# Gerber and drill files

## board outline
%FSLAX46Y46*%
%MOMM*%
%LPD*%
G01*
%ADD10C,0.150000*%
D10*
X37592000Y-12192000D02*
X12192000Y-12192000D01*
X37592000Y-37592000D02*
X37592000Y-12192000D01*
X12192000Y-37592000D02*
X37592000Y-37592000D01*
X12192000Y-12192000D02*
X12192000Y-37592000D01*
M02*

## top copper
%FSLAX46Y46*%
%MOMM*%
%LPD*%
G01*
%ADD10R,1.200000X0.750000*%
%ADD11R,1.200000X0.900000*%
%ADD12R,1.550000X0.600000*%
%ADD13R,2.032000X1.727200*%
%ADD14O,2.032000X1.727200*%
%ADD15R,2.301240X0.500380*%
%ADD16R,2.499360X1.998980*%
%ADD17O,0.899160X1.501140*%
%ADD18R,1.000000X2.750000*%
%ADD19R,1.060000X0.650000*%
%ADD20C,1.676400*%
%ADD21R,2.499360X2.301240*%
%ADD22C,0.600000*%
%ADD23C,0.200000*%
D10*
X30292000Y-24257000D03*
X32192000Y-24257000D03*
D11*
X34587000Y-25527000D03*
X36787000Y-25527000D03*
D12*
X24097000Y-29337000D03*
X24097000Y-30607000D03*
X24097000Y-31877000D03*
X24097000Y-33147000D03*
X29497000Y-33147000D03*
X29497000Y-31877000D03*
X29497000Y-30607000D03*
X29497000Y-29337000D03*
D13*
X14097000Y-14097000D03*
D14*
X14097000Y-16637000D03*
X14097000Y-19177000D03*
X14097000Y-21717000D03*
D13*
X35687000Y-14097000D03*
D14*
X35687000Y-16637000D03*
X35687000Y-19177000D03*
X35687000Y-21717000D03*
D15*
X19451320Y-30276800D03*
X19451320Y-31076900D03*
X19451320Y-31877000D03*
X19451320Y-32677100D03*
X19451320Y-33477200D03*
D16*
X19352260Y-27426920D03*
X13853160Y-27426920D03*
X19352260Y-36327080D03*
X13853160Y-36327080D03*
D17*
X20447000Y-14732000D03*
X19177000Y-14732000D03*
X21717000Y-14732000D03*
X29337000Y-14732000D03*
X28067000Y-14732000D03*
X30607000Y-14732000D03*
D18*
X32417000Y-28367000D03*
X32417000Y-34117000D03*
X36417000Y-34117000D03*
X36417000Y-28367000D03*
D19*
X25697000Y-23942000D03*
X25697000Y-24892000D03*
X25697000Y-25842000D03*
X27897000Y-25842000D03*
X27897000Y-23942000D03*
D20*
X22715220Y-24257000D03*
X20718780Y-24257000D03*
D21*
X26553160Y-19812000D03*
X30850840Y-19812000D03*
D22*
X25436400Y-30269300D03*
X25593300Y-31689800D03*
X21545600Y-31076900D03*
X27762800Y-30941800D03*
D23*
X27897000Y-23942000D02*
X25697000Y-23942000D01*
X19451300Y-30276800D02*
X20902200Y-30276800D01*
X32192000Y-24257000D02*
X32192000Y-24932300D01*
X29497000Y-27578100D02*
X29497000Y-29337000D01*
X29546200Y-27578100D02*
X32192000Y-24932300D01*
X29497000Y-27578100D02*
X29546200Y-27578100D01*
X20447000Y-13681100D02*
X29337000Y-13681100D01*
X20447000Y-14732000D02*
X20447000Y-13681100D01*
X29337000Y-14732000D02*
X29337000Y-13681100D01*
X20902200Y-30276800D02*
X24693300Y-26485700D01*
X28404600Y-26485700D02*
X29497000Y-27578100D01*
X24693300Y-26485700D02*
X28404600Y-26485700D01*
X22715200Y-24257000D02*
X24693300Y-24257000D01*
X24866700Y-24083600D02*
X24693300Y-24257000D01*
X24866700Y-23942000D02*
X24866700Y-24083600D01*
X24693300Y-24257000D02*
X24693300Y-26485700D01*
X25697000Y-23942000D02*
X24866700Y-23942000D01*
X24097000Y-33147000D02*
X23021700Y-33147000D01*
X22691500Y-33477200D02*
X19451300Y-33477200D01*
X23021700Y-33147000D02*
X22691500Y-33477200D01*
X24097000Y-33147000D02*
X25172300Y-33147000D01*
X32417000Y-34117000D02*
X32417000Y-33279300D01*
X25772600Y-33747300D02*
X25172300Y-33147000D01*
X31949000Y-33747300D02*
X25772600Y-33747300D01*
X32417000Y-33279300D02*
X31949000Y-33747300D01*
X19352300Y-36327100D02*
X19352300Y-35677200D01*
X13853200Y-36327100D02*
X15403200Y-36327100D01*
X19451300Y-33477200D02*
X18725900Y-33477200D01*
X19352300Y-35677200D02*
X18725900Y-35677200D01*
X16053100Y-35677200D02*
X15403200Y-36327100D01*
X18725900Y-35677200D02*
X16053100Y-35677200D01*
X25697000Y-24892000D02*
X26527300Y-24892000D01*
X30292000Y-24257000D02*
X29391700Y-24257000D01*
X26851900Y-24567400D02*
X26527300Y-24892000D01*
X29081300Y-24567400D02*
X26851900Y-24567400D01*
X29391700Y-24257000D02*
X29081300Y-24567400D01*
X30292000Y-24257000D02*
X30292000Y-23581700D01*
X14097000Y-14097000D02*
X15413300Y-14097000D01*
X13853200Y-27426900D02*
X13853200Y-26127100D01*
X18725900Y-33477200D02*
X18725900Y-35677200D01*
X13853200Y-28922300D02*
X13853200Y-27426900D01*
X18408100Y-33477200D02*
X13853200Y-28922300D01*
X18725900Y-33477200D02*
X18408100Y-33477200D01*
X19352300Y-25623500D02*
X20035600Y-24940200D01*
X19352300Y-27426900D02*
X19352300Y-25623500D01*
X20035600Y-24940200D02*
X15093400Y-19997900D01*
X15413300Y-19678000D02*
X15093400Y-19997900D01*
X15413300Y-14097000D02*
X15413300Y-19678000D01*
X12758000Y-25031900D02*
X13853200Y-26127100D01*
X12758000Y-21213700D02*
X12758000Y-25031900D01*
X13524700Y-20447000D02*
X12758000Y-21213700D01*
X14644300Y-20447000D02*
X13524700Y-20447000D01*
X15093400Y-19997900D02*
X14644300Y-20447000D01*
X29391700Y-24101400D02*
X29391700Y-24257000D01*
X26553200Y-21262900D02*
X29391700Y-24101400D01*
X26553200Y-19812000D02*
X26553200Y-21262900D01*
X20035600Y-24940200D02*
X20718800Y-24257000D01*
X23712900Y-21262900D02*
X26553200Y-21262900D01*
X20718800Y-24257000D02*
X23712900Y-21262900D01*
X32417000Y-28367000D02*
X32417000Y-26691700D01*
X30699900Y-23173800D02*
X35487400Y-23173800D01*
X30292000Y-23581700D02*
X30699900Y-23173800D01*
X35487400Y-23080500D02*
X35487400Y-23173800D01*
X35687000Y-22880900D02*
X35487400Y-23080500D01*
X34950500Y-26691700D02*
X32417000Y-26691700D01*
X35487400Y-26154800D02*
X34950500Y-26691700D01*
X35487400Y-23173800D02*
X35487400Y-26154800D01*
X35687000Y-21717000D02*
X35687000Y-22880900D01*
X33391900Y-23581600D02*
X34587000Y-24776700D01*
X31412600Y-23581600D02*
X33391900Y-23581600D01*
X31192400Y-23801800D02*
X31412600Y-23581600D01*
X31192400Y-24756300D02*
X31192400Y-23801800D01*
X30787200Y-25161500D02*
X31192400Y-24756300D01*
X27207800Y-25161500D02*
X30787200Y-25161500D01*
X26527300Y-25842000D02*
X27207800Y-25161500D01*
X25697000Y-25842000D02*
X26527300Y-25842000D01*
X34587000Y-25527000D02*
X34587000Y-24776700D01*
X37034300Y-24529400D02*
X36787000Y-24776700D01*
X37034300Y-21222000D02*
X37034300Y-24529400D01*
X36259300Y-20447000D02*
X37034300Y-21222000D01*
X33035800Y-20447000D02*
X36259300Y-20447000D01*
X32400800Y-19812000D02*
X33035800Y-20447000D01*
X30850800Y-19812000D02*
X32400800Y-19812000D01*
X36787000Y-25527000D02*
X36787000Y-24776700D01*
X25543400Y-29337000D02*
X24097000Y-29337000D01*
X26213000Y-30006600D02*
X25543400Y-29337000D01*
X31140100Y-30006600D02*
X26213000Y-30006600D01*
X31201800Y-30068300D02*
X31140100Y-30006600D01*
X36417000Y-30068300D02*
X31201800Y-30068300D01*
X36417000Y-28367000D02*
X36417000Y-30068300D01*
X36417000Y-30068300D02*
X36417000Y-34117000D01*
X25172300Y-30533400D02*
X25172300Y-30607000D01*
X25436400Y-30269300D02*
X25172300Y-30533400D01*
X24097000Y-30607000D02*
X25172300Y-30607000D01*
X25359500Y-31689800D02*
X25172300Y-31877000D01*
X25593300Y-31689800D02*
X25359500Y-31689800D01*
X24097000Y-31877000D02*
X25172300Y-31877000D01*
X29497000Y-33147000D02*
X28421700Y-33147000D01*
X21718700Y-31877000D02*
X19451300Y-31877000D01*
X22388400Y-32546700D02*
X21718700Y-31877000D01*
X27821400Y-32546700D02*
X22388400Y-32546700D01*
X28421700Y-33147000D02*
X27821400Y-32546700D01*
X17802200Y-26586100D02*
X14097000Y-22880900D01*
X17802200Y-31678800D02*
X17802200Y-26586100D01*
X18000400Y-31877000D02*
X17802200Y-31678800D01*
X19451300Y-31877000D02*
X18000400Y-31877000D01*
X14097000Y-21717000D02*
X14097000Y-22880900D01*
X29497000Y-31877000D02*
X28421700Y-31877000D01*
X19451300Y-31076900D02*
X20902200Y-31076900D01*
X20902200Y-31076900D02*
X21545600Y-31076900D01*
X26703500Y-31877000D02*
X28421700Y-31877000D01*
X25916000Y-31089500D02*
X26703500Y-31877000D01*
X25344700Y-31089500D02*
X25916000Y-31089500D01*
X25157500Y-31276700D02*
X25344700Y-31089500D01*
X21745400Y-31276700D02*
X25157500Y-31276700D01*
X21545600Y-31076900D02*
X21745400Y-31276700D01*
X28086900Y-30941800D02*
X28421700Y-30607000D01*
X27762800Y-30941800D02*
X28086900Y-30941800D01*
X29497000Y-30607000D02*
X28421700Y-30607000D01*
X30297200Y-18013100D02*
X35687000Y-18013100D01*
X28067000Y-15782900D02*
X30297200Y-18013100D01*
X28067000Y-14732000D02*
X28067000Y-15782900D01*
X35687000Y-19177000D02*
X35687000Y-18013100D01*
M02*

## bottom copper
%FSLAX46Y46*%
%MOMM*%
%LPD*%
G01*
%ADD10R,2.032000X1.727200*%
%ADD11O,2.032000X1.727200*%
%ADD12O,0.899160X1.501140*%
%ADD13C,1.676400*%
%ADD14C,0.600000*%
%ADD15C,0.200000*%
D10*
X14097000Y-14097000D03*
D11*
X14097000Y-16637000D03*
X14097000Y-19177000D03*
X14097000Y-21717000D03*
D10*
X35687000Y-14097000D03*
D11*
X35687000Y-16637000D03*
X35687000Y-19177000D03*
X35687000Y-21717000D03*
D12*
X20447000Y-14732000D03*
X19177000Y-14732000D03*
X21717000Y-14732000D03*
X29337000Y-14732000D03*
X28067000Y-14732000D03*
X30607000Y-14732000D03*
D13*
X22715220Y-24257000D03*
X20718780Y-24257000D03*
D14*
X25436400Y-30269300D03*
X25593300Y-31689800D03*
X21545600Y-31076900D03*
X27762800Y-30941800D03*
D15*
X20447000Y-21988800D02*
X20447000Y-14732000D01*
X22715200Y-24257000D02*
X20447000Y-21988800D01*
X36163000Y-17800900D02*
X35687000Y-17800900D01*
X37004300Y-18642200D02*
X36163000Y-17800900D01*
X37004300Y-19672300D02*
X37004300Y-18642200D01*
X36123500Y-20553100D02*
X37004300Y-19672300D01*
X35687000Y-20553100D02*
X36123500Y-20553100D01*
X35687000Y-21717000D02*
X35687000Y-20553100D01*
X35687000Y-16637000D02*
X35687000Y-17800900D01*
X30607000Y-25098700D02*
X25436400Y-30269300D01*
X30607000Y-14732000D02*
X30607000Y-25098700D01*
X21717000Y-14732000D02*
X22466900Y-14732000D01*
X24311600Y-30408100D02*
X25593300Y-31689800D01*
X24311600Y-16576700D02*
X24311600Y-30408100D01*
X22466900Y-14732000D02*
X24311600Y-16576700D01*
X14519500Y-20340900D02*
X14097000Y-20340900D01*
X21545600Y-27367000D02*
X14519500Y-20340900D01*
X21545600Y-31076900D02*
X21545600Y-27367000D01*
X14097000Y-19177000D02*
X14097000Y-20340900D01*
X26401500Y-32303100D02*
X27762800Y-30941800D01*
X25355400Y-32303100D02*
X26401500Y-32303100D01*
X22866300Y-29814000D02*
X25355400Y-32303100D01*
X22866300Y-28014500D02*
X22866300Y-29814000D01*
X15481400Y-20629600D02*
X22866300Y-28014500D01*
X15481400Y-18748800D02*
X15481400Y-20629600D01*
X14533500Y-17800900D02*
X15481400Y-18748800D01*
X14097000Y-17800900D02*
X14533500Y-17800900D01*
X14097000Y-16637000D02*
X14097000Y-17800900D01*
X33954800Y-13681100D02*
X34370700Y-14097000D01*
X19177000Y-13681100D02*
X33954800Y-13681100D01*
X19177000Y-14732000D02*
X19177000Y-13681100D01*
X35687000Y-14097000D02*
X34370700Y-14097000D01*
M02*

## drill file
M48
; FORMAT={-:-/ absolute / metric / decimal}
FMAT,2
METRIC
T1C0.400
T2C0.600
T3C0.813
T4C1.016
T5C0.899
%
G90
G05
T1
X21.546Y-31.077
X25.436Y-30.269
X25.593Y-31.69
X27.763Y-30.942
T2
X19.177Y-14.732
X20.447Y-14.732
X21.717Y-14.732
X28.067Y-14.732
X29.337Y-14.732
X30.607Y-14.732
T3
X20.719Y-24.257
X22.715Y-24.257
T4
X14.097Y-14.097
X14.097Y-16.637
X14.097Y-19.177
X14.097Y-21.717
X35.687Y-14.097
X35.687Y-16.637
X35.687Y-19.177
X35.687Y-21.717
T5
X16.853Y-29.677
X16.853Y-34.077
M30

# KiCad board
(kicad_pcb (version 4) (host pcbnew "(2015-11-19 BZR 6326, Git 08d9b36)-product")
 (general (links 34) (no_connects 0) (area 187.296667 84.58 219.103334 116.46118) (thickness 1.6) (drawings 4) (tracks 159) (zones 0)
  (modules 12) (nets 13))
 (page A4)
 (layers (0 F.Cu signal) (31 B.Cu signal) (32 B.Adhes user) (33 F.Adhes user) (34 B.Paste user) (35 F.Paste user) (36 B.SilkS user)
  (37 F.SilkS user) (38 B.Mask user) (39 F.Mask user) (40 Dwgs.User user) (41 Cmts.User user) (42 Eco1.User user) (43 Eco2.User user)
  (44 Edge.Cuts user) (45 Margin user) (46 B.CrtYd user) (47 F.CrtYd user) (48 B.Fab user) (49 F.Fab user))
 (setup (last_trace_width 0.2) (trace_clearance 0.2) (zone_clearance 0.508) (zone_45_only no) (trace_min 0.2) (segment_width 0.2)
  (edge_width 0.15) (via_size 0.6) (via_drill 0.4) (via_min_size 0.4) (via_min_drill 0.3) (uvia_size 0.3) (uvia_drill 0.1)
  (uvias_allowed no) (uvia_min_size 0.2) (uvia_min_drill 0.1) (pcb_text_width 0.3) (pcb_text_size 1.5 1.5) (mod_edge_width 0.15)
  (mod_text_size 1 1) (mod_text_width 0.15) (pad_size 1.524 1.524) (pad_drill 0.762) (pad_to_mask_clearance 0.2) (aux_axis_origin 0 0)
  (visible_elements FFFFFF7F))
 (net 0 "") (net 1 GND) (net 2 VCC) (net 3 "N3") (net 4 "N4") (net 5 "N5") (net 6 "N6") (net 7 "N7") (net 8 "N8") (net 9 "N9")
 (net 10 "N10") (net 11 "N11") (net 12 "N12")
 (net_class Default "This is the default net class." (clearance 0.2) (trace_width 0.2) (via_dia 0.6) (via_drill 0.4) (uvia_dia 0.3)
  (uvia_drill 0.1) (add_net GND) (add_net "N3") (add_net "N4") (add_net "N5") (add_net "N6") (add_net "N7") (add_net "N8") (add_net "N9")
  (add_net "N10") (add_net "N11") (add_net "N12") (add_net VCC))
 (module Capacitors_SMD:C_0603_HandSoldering (layer F.Cu) (at 31.242 24.257)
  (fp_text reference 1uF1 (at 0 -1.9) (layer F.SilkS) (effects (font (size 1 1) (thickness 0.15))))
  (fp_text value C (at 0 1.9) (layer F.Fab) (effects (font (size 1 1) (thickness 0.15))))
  (pad 1 smd rect (at -0.95 0) (size 1.2 0.75) (layers F.Cu F.Paste F.Mask) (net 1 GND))
  (pad 2 smd rect (at 0.95 0) (size 1.2 0.75) (layers F.Cu F.Paste F.Mask) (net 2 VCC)))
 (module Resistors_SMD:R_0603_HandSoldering (layer F.Cu) (at 35.687 25.527)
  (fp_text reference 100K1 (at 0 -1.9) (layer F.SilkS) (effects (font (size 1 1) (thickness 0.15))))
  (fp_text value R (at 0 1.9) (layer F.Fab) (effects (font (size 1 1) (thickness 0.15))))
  (pad 1 smd rect (at -1.1 0) (size 1.2 0.9) (layers F.Cu F.Paste F.Mask) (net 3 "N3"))
  (pad 2 smd rect (at 1.1 0) (size 1.2 0.9) (layers F.Cu F.Paste F.Mask) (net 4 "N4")))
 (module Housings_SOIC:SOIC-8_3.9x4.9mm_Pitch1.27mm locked (layer F.Cu) (at 26.797 31.242)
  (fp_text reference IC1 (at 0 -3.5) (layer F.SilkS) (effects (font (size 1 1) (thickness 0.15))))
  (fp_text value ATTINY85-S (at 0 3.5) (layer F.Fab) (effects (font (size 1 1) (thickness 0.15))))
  (pad 1 smd rect (at -2.7 -1.905) (size 1.55 0.6) (layers F.Cu F.Paste F.Mask) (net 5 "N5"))
  (pad 2 smd rect (at -2.7 -0.635) (size 1.55 0.6) (layers F.Cu F.Paste F.Mask) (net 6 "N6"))
  (pad 3 smd rect (at -2.7 0.635) (size 1.55 0.6) (layers F.Cu F.Paste F.Mask) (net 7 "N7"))
  (pad 4 smd rect (at -2.7 1.905) (size 1.55 0.6) (layers F.Cu F.Paste F.Mask) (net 1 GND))
  (pad 5 smd rect (at 2.7 1.905) (size 1.55 0.6) (layers F.Cu F.Paste F.Mask) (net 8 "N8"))
  (pad 6 smd rect (at 2.7 0.635) (size 1.55 0.6) (layers F.Cu F.Paste F.Mask) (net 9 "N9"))
  (pad 7 smd rect (at 2.7 -0.635) (size 1.55 0.6) (layers F.Cu F.Paste F.Mask) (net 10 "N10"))
  (pad 8 smd rect (at 2.7 -1.905) (size 1.55 0.6) (layers F.Cu F.Paste F.Mask) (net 2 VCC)))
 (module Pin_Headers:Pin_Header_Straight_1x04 (layer F.Cu) (at 14.097 14.097)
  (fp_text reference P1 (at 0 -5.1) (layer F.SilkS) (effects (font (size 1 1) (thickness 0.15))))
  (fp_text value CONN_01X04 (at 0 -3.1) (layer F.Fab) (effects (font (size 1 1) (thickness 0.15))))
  (pad 1 thru_hole rect (at 0 0) (size 2.032 1.7272) (drill 1.016) (layers *.Cu *.Mask F.SilkS) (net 1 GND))
  (pad 2 thru_hole oval (at 0 2.54) (size 2.032 1.7272) (drill 1.016) (layers *.Cu *.Mask F.SilkS) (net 10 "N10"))
  (pad 3 thru_hole oval (at 0 5.08) (size 2.032 1.7272) (drill 1.016) (layers *.Cu *.Mask F.SilkS) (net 9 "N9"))
  (pad 4 thru_hole oval (at 0 7.62) (size 2.032 1.7272) (drill 1.016) (layers *.Cu *.Mask F.SilkS) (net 8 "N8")))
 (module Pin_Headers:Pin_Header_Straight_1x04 (layer F.Cu) (at 35.687 14.097)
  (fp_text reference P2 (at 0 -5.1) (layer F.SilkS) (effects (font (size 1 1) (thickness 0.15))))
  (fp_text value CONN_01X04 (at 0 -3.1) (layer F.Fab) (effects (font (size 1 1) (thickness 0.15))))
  (pad 1 thru_hole rect (at 0 0) (size 2.032 1.7272) (drill 1.016) (layers *.Cu *.Mask F.SilkS) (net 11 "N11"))
  (pad 2 thru_hole oval (at 0 2.54) (size 2.032 1.7272) (drill 1.016) (layers *.Cu *.Mask F.SilkS) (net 1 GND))
  (pad 3 thru_hole oval (at 0 5.08) (size 2.032 1.7272) (drill 1.016) (layers *.Cu *.Mask F.SilkS) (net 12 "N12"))
  (pad 4 thru_hole oval (at 0 7.62) (size 2.032 1.7272) (drill 1.016) (layers *.Cu *.Mask F.SilkS) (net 1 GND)))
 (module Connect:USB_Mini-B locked (layer F.Cu) (at 16.002 31.877)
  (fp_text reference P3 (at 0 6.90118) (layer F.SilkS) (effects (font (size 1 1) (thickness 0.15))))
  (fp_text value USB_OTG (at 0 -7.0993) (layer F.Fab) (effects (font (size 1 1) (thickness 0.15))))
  (pad 1 smd rect (at 3.44932 -1.6002) (size 2.30124 0.50038) (layers F.Cu F.Paste F.Mask) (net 2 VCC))
  (pad 2 smd rect (at 3.44932 -0.8001) (size 2.30124 0.50038) (layers F.Cu F.Paste F.Mask) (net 9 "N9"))
  (pad 3 smd rect (at 3.44932 0) (size 2.30124 0.50038) (layers F.Cu F.Paste F.Mask) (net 8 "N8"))
  (pad 4 smd rect (at 3.44932 0.8001) (size 2.30124 0.50038) (layers F.Cu F.Paste F.Mask))
  (pad 5 smd rect (at 3.44932 1.6002) (size 2.30124 0.50038) (layers F.Cu F.Paste F.Mask) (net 1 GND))
  (pad 6 smd rect (at 3.35026 -4.45008) (size 2.49936 1.99898) (layers F.Cu F.Paste F.Mask) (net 1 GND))
  (pad 6 smd rect (at -2.14884 -4.45008) (size 2.49936 1.99898) (layers F.Cu F.Paste F.Mask) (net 1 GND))
  (pad 6 smd rect (at 3.35026 4.45008) (size 2.49936 1.99898) (layers F.Cu F.Paste F.Mask) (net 1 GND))
  (pad 6 smd rect (at -2.14884 4.45008) (size 2.49936 1.99898) (layers F.Cu F.Paste F.Mask) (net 1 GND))
  (pad "" np_thru_hole circle (at 0.8509 -2.19964) (size 0.89916 0.89916) (drill 0.89916) (layers *.Cu *.Mask F.SilkS))
  (pad "" np_thru_hole circle (at 0.8509 2.19964) (size 0.89916 0.89916) (drill 0.89916) (layers *.Cu *.Mask F.SilkS)))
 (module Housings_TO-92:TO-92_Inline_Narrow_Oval (layer F.Cu) (at 21.717 14.732 180)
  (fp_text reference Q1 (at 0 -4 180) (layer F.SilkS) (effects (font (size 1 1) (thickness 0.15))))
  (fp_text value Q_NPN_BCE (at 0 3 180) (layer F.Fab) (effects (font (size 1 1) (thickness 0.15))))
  (pad 2 thru_hole oval (at 1.27 0) (size 0.89916 1.50114) (drill 0.6) (layers *.Cu *.Mask F.SilkS) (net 2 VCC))
  (pad 3 thru_hole oval (at 2.54 0) (size 0.89916 1.50114) (drill 0.6) (layers *.Cu *.Mask F.SilkS) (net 11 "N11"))
  (pad 1 thru_hole oval (at 0 0) (size 0.89916 1.50114) (drill 0.6) (layers *.Cu *.Mask F.SilkS) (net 7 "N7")))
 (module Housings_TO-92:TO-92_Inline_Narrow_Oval (layer F.Cu) (at 30.607 14.732 180)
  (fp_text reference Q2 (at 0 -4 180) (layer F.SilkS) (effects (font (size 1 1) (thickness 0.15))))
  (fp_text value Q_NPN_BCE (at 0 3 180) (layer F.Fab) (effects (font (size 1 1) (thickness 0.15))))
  (pad 2 thru_hole oval (at 1.27 0) (size 0.89916 1.50114) (drill 0.6) (layers *.Cu *.Mask F.SilkS) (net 2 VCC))
  (pad 3 thru_hole oval (at 2.54 0) (size 0.89916 1.50114) (drill 0.6) (layers *.Cu *.Mask F.SilkS) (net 12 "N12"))
  (pad 1 thru_hole oval (at 0 0) (size 0.89916 1.50114) (drill 0.6) (layers *.Cu *.Mask F.SilkS) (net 6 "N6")))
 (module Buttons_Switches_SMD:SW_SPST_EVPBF (layer F.Cu) (at 34.417 31.242 90)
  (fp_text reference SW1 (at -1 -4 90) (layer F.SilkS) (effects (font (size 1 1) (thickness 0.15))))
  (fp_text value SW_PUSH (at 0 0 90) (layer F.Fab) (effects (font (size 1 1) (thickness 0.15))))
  (pad 1 smd rect (at 2.875 -2 90) (size 2.75 1) (layers F.Cu F.Paste F.Mask) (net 1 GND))
  (pad 1 smd rect (at -2.875 -2 90) (size 2.75 1) (layers F.Cu F.Paste F.Mask) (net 1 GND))
  (pad 2 smd rect (at -2.875 2 90) (size 2.75 1) (layers F.Cu F.Paste F.Mask) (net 5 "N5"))
  (pad 2 smd rect (at 2.875 2 90) (size 2.75 1) (layers F.Cu F.Paste F.Mask) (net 5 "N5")))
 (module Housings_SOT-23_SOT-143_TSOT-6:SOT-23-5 (layer F.Cu) (at 26.797 24.892)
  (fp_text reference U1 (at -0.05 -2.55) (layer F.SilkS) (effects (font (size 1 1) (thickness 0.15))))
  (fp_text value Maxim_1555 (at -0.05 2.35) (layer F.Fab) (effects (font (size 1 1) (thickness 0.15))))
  (pad 1 smd rect (at -1.1 -0.95) (size 1.06 0.65) (layers F.Cu F.Paste F.Mask) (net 2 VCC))
  (pad 2 smd rect (at -1.1 0) (size 1.06 0.65) (layers F.Cu F.Paste F.Mask) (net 1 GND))
  (pad 3 smd rect (at -1.1 0.95) (size 1.06 0.65) (layers F.Cu F.Paste F.Mask) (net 3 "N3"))
  (pad 4 smd rect (at 1.1 0.95) (size 1.06 0.65) (layers F.Cu F.Paste F.Mask))
  (pad 5 smd rect (at 1.1 -0.95) (size 1.06 0.65) (layers F.Cu F.Paste F.Mask) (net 2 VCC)))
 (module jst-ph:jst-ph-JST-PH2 (layer F.Cu) (at 21.717 24.257)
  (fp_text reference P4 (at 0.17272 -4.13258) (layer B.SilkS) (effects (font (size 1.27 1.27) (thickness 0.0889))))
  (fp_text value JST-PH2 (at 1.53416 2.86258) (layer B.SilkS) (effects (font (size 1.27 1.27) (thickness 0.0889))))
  (pad 1 thru_hole circle (at 0.99822 0) (size 1.6764 3.3528) (drill 0.8128) (layers *.Cu F.Paste F.SilkS F.Mask) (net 2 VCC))
  (pad 2 thru_hole circle (at -0.99822 0) (size 1.6764 3.3528) (drill 0.8128) (layers *.Cu F.Paste F.SilkS F.Mask) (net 1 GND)))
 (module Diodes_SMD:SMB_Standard (layer F.Cu) (at 28.702 19.812)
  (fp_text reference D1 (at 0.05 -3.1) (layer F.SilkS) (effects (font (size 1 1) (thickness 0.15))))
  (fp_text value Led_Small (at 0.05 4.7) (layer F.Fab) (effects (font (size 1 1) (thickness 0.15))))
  (pad 1 smd rect (at -2.14884 0) (size 2.49936 2.30124) (layers F.Cu F.Paste F.Mask) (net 1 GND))
  (pad 2 smd rect (at 2.14884 0) (size 2.49936 2.30124) (layers F.Cu F.Paste F.Mask) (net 4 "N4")))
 (gr_line (start 37.592 12.192) (end 12.192 12.192) (angle 90) (layer Edge.Cuts) (width 0.15))
 (gr_line (start 37.592 37.592) (end 37.592 12.192) (angle 90) (layer Edge.Cuts) (width 0.15))
 (gr_line (start 12.192 37.592) (end 37.592 37.592) (angle 90) (layer Edge.Cuts) (width 0.15))
 (gr_line (start 12.192 12.192) (end 12.192 37.592) (angle 90) (layer Edge.Cuts) (width 0.15))
 (segment (start 20.447 21.9888) (end 20.447 14.732) (width 0.2) (layer B.Cu) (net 2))
 (segment (start 22.7152 24.257) (end 20.447 21.9888) (width 0.2) (layer B.Cu) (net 2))
 (segment (start 27.897 23.942) (end 25.697 23.942) (width 0.2) (layer F.Cu) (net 2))
 (segment (start 19.4513 30.2768) (end 20.9022 30.2768) (width 0.2) (layer F.Cu) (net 2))
 (segment (start 32.192 24.257) (end 32.192 24.9323) (width 0.2) (layer F.Cu) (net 2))
 (segment (start 29.497 27.5781) (end 29.497 29.337) (width 0.2) (layer F.Cu) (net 2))
 (segment (start 29.5462 27.5781) (end 32.192 24.9323) (width 0.2) (layer F.Cu) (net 2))
 (segment (start 29.497 27.5781) (end 29.5462 27.5781) (width 0.2) (layer F.Cu) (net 2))
 (segment (start 20.447 13.6811) (end 29.337 13.6811) (width 0.2) (layer F.Cu) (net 2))
 (segment (start 20.447 14.732) (end 20.447 13.6811) (width 0.2) (layer F.Cu) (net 2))
 (segment (start 29.337 14.732) (end 29.337 13.6811) (width 0.2) (layer F.Cu) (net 2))
 (segment (start 20.9022 30.2768) (end 24.6933 26.4857) (width 0.2) (layer F.Cu) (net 2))
 (segment (start 28.4046 26.4857) (end 29.497 27.5781) (width 0.2) (layer F.Cu) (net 2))
 (segment (start 24.6933 26.4857) (end 28.4046 26.4857) (width 0.2) (layer F.Cu) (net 2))
 (segment (start 22.7152 24.257) (end 24.6933 24.257) (width 0.2) (layer F.Cu) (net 2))
 (segment (start 24.8667 24.0836) (end 24.6933 24.257) (width 0.2) (layer F.Cu) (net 2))
 (segment (start 24.8667 23.942) (end 24.8667 24.0836) (width 0.2) (layer F.Cu) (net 2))
 (segment (start 24.6933 24.257) (end 24.6933 26.4857) (width 0.2) (layer F.Cu) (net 2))
 (segment (start 25.697 23.942) (end 24.8667 23.942) (width 0.2) (layer F.Cu) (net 2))
 (segment (start 24.097 33.147) (end 23.0217 33.147) (width 0.2) (layer F.Cu) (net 1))
 (segment (start 22.6915 33.4772) (end 19.4513 33.4772) (width 0.2) (layer F.Cu) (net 1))
 (segment (start 23.0217 33.147) (end 22.6915 33.4772) (width 0.2) (layer F.Cu) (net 1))
 (segment (start 24.097 33.147) (end 25.1723 33.147) (width 0.2) (layer F.Cu) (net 1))
 (segment (start 32.417 34.117) (end 32.417 33.2793) (width 0.2) (layer F.Cu) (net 1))
 (segment (start 25.7726 33.7473) (end 25.1723 33.147) (width 0.2) (layer F.Cu) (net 1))
 (segment (start 31.949 33.7473) (end 25.7726 33.7473) (width 0.2) (layer F.Cu) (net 1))
 (segment (start 32.417 33.2793) (end 31.949 33.7473) (width 0.2) (layer F.Cu) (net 1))
 (segment (start 36.163 17.8009) (end 35.687 17.8009) (width 0.2) (layer B.Cu) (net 1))
 (segment (start 37.0043 18.6422) (end 36.163 17.8009) (width 0.2) (layer B.Cu) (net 1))
 (segment (start 37.0043 19.6723) (end 37.0043 18.6422) (width 0.2) (layer B.Cu) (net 1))
 (segment (start 36.1235 20.5531) (end 37.0043 19.6723) (width 0.2) (layer B.Cu) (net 1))
 (segment (start 35.687 20.5531) (end 36.1235 20.5531) (width 0.2) (layer B.Cu) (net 1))
 (segment (start 35.687 21.717) (end 35.687 20.5531) (width 0.2) (layer B.Cu) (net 1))
 (segment (start 35.687 16.637) (end 35.687 17.8009) (width 0.2) (layer B.Cu) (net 1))
 (segment (start 19.3523 36.3271) (end 19.3523 35.6772) (width 0.2) (layer F.Cu) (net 1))
 (segment (start 13.8532 36.3271) (end 15.4032 36.3271) (width 0.2) (layer F.Cu) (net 1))
 (segment (start 19.4513 33.4772) (end 18.7259 33.4772) (width 0.2) (layer F.Cu) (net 1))
 (segment (start 19.3523 35.6772) (end 18.7259 35.6772) (width 0.2) (layer F.Cu) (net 1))
 (segment (start 16.0531 35.6772) (end 15.4032 36.3271) (width 0.2) (layer F.Cu) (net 1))
 (segment (start 18.7259 35.6772) (end 16.0531 35.6772) (width 0.2) (layer F.Cu) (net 1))
 (segment (start 25.697 24.892) (end 26.5273 24.892) (width 0.2) (layer F.Cu) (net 1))
 (segment (start 30.292 24.257) (end 29.3917 24.257) (width 0.2) (layer F.Cu) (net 1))
 (segment (start 26.8519 24.5674) (end 26.5273 24.892) (width 0.2) (layer F.Cu) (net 1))
 (segment (start 29.0813 24.5674) (end 26.8519 24.5674) (width 0.2) (layer F.Cu) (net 1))
 (segment (start 29.3917 24.257) (end 29.0813 24.5674) (width 0.2) (layer F.Cu) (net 1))
 (segment (start 30.292 24.257) (end 30.292 23.5817) (width 0.2) (layer F.Cu) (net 1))
 (segment (start 14.097 14.097) (end 15.4133 14.097) (width 0.2) (layer F.Cu) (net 1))
 (segment (start 13.8532 27.4269) (end 13.8532 26.1271) (width 0.2) (layer F.Cu) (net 1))
 (segment (start 18.7259 33.4772) (end 18.7259 35.6772) (width 0.2) (layer F.Cu) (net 1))
 (segment (start 13.8532 28.9223) (end 13.8532 27.4269) (width 0.2) (layer F.Cu) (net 1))
 (segment (start 18.4081 33.4772) (end 13.8532 28.9223) (width 0.2) (layer F.Cu) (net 1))
 (segment (start 18.7259 33.4772) (end 18.4081 33.4772) (width 0.2) (layer F.Cu) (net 1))
 (segment (start 19.3523 25.6235) (end 20.0356 24.9402) (width 0.2) (layer F.Cu) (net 1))
 (segment (start 19.3523 27.4269) (end 19.3523 25.6235) (width 0.2) (layer F.Cu) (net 1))
 (segment (start 20.0356 24.9402) (end 15.0934 19.9979) (width 0.2) (layer F.Cu) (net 1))
 (segment (start 15.4133 19.678) (end 15.0934 19.9979) (width 0.2) (layer F.Cu) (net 1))
 (segment (start 15.4133 14.097) (end 15.4133 19.678) (width 0.2) (layer F.Cu) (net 1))
 (segment (start 12.758 25.0319) (end 13.8532 26.1271) (width 0.2) (layer F.Cu) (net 1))
 (segment (start 12.758 21.2137) (end 12.758 25.0319) (width 0.2) (layer F.Cu) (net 1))
 (segment (start 13.5247 20.447) (end 12.758 21.2137) (width 0.2) (layer F.Cu) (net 1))
 (segment (start 14.6443 20.447) (end 13.5247 20.447) (width 0.2) (layer F.Cu) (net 1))
 (segment (start 15.0934 19.9979) (end 14.6443 20.447) (width 0.2) (layer F.Cu) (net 1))
 (segment (start 29.3917 24.1014) (end 29.3917 24.257) (width 0.2) (layer F.Cu) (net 1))
 (segment (start 26.5532 21.2629) (end 29.3917 24.1014) (width 0.2) (layer F.Cu) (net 1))
 (segment (start 26.5532 19.812) (end 26.5532 21.2629) (width 0.2) (layer F.Cu) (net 1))
 (segment (start 20.0356 24.9402) (end 20.7188 24.257) (width 0.2) (layer F.Cu) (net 1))
 (segment (start 23.7129 21.2629) (end 26.5532 21.2629) (width 0.2) (layer F.Cu) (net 1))
 (segment (start 20.7188 24.257) (end 23.7129 21.2629) (width 0.2) (layer F.Cu) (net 1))
 (segment (start 32.417 28.367) (end 32.417 26.6917) (width 0.2) (layer F.Cu) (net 1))
 (segment (start 30.6999 23.1738) (end 35.4874 23.1738) (width 0.2) (layer F.Cu) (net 1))
 (segment (start 30.292 23.5817) (end 30.6999 23.1738) (width 0.2) (layer F.Cu) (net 1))
 (segment (start 35.4874 23.0805) (end 35.4874 23.1738) (width 0.2) (layer F.Cu) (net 1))
 (segment (start 35.687 22.8809) (end 35.4874 23.0805) (width 0.2) (layer F.Cu) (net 1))
 (segment (start 34.9505 26.6917) (end 32.417 26.6917) (width 0.2) (layer F.Cu) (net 1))
 (segment (start 35.4874 26.1548) (end 34.9505 26.6917) (width 0.2) (layer F.Cu) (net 1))
 (segment (start 35.4874 23.1738) (end 35.4874 26.1548) (width 0.2) (layer F.Cu) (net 1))
 (segment (start 35.687 21.717) (end 35.687 22.8809) (width 0.2) (layer F.Cu) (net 1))
 (segment (start 33.3919 23.5816) (end 34.587 24.7767) (width 0.2) (layer F.Cu) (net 3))
 (segment (start 31.4126 23.5816) (end 33.3919 23.5816) (width 0.2) (layer F.Cu) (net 3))
 (segment (start 31.1924 23.8018) (end 31.4126 23.5816) (width 0.2) (layer F.Cu) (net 3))
 (segment (start 31.1924 24.7563) (end 31.1924 23.8018) (width 0.2) (layer F.Cu) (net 3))
 (segment (start 30.7872 25.1615) (end 31.1924 24.7563) (width 0.2) (layer F.Cu) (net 3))
 (segment (start 27.2078 25.1615) (end 30.7872 25.1615) (width 0.2) (layer F.Cu) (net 3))
 (segment (start 26.5273 25.842) (end 27.2078 25.1615) (width 0.2) (layer F.Cu) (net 3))
 (segment (start 25.697 25.842) (end 26.5273 25.842) (width 0.2) (layer F.Cu) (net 3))
 (segment (start 34.587 25.527) (end 34.587 24.7767) (width 0.2) (layer F.Cu) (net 3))
 (segment (start 37.0343 24.5294) (end 36.787 24.7767) (width 0.2) (layer F.Cu) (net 4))
 (segment (start 37.0343 21.222) (end 37.0343 24.5294) (width 0.2) (layer F.Cu) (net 4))
 (segment (start 36.2593 20.447) (end 37.0343 21.222) (width 0.2) (layer F.Cu) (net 4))
 (segment (start 33.0358 20.447) (end 36.2593 20.447) (width 0.2) (layer F.Cu) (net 4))
 (segment (start 32.4008 19.812) (end 33.0358 20.447) (width 0.2) (layer F.Cu) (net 4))
 (segment (start 30.8508 19.812) (end 32.4008 19.812) (width 0.2) (layer F.Cu) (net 4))
 (segment (start 36.787 25.527) (end 36.787 24.7767) (width 0.2) (layer F.Cu) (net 4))
 (segment (start 25.5434 29.337) (end 24.097 29.337) (width 0.2) (layer F.Cu) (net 5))
 (segment (start 26.213 30.0066) (end 25.5434 29.337) (width 0.2) (layer F.Cu) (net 5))
 (segment (start 31.1401 30.0066) (end 26.213 30.0066) (width 0.2) (layer F.Cu) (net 5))
 (segment (start 31.2018 30.0683) (end 31.1401 30.0066) (width 0.2) (layer F.Cu) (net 5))
 (segment (start 36.417 30.0683) (end 31.2018 30.0683) (width 0.2) (layer F.Cu) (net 5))
 (segment (start 36.417 28.367) (end 36.417 30.0683) (width 0.2) (layer F.Cu) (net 5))
 (segment (start 36.417 30.0683) (end 36.417 34.117) (width 0.2) (layer F.Cu) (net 5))
 (via (at 25.4364 30.2693) (size 0.6) (layers F.Cu B.Cu) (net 6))
 (segment (start 30.607 25.0987) (end 25.4364 30.2693) (width 0.2) (layer B.Cu) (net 6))
 (segment (start 30.607 14.732) (end 30.607 25.0987) (width 0.2) (layer B.Cu) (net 6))
 (segment (start 25.1723 30.5334) (end 25.1723 30.607) (width 0.2) (layer F.Cu) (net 6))
 (segment (start 25.4364 30.2693) (end 25.1723 30.5334) (width 0.2) (layer F.Cu) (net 6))
 (segment (start 24.097 30.607) (end 25.1723 30.607) (width 0.2) (layer F.Cu) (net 6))
 (via (at 25.5933 31.6898) (size 0.6) (layers F.Cu B.Cu) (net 7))
 (segment (start 25.3595 31.6898) (end 25.1723 31.877) (width 0.2) (layer F.Cu) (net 7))
 (segment (start 25.5933 31.6898) (end 25.3595 31.6898) (width 0.2) (layer F.Cu) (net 7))
 (segment (start 24.097 31.877) (end 25.1723 31.877) (width 0.2) (layer F.Cu) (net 7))
 (segment (start 21.717 14.732) (end 22.4669 14.732) (width 0.2) (layer B.Cu) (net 7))
 (segment (start 24.3116 30.4081) (end 25.5933 31.6898) (width 0.2) (layer B.Cu) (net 7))
 (segment (start 24.3116 16.5767) (end 24.3116 30.4081) (width 0.2) (layer B.Cu) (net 7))
 (segment (start 22.4669 14.732) (end 24.3116 16.5767) (width 0.2) (layer B.Cu) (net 7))
 (segment (start 29.497 33.147) (end 28.4217 33.147) (width 0.2) (layer F.Cu) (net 8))
 (segment (start 21.7187 31.877) (end 19.4513 31.877) (width 0.2) (layer F.Cu) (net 8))
 (segment (start 22.3884 32.5467) (end 21.7187 31.877) (width 0.2) (layer F.Cu) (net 8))
 (segment (start 27.8214 32.5467) (end 22.3884 32.5467) (width 0.2) (layer F.Cu) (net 8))
 (segment (start 28.4217 33.147) (end 27.8214 32.5467) (width 0.2) (layer F.Cu) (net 8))
 (segment (start 17.8022 26.5861) (end 14.097 22.8809) (width 0.2) (layer F.Cu) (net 8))
 (segment (start 17.8022 31.6788) (end 17.8022 26.5861) (width 0.2) (layer F.Cu) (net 8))
 (segment (start 18.0004 31.877) (end 17.8022 31.6788) (width 0.2) (layer F.Cu) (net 8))
 (segment (start 19.4513 31.877) (end 18.0004 31.877) (width 0.2) (layer F.Cu) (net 8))
 (segment (start 14.097 21.717) (end 14.097 22.8809) (width 0.2) (layer F.Cu) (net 8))
 (via (at 21.5456 31.0769) (size 0.6) (layers F.Cu B.Cu) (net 9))
 (segment (start 29.497 31.877) (end 28.4217 31.877) (width 0.2) (layer F.Cu) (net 9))
 (segment (start 19.4513 31.0769) (end 20.9022 31.0769) (width 0.2) (layer F.Cu) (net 9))
 (segment (start 20.9022 31.0769) (end 21.5456 31.0769) (width 0.2) (layer F.Cu) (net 9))
 (segment (start 14.5195 20.3409) (end 14.097 20.3409) (width 0.2) (layer B.Cu) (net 9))
 (segment (start 21.5456 27.367) (end 14.5195 20.3409) (width 0.2) (layer B.Cu) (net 9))
 (segment (start 21.5456 31.0769) (end 21.5456 27.367) (width 0.2) (layer B.Cu) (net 9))
 (segment (start 14.097 19.177) (end 14.097 20.3409) (width 0.2) (layer B.Cu) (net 9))
 (segment (start 26.7035 31.877) (end 28.4217 31.877) (width 0.2) (layer F.Cu) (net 9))
 (segment (start 25.916 31.0895) (end 26.7035 31.877) (width 0.2) (layer F.Cu) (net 9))
 (segment (start 25.3447 31.0895) (end 25.916 31.0895) (width 0.2) (layer F.Cu) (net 9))
 (segment (start 25.1575 31.2767) (end 25.3447 31.0895) (width 0.2) (layer F.Cu) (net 9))
 (segment (start 21.7454 31.2767) (end 25.1575 31.2767) (width 0.2) (layer F.Cu) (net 9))
 (segment (start 21.5456 31.0769) (end 21.7454 31.2767) (width 0.2) (layer F.Cu) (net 9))
 (via (at 27.7628 30.9418) (size 0.6) (layers F.Cu B.Cu) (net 10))
 (segment (start 26.4015 32.3031) (end 27.7628 30.9418) (width 0.2) (layer B.Cu) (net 10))
 (segment (start 25.3554 32.3031) (end 26.4015 32.3031) (width 0.2) (layer B.Cu) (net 10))
 (segment (start 22.8663 29.814) (end 25.3554 32.3031) (width 0.2) (layer B.Cu) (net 10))
 (segment (start 22.8663 28.0145) (end 22.8663 29.814) (width 0.2) (layer B.Cu) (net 10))
 (segment (start 15.4814 20.6296) (end 22.8663 28.0145) (width 0.2) (layer B.Cu) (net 10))
 (segment (start 15.4814 18.7488) (end 15.4814 20.6296) (width 0.2) (layer B.Cu) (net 10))
 (segment (start 14.5335 17.8009) (end 15.4814 18.7488) (width 0.2) (layer B.Cu) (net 10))
 (segment (start 14.097 17.8009) (end 14.5335 17.8009) (width 0.2) (layer B.Cu) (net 10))
 (segment (start 28.0869 30.9418) (end 28.4217 30.607) (width 0.2) (layer F.Cu) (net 10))
 (segment (start 27.7628 30.9418) (end 28.0869 30.9418) (width 0.2) (layer F.Cu) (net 10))
 (segment (start 29.497 30.607) (end 28.4217 30.607) (width 0.2) (layer F.Cu) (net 10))
 (segment (start 14.097 16.637) (end 14.097 17.8009) (width 0.2) (layer B.Cu) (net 10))
 (segment (start 33.9548 13.6811) (end 34.3707 14.097) (width 0.2) (layer B.Cu) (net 11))
 (segment (start 19.177 13.6811) (end 33.9548 13.6811) (width 0.2) (layer B.Cu) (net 11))
 (segment (start 19.177 14.732) (end 19.177 13.6811) (width 0.2) (layer B.Cu) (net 11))
 (segment (start 35.687 14.097) (end 34.3707 14.097) (width 0.2) (layer B.Cu) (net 11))
 (segment (start 30.2972 18.0131) (end 35.687 18.0131) (width 0.2) (layer F.Cu) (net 12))
 (segment (start 28.067 15.7829) (end 30.2972 18.0131) (width 0.2) (layer F.Cu) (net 12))
 (segment (start 28.067 14.732) (end 28.067 15.7829) (width 0.2) (layer F.Cu) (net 12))
 (segment (start 35.687 19.177) (end 35.687 18.0131) (width 0.2) (layer F.Cu) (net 12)))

